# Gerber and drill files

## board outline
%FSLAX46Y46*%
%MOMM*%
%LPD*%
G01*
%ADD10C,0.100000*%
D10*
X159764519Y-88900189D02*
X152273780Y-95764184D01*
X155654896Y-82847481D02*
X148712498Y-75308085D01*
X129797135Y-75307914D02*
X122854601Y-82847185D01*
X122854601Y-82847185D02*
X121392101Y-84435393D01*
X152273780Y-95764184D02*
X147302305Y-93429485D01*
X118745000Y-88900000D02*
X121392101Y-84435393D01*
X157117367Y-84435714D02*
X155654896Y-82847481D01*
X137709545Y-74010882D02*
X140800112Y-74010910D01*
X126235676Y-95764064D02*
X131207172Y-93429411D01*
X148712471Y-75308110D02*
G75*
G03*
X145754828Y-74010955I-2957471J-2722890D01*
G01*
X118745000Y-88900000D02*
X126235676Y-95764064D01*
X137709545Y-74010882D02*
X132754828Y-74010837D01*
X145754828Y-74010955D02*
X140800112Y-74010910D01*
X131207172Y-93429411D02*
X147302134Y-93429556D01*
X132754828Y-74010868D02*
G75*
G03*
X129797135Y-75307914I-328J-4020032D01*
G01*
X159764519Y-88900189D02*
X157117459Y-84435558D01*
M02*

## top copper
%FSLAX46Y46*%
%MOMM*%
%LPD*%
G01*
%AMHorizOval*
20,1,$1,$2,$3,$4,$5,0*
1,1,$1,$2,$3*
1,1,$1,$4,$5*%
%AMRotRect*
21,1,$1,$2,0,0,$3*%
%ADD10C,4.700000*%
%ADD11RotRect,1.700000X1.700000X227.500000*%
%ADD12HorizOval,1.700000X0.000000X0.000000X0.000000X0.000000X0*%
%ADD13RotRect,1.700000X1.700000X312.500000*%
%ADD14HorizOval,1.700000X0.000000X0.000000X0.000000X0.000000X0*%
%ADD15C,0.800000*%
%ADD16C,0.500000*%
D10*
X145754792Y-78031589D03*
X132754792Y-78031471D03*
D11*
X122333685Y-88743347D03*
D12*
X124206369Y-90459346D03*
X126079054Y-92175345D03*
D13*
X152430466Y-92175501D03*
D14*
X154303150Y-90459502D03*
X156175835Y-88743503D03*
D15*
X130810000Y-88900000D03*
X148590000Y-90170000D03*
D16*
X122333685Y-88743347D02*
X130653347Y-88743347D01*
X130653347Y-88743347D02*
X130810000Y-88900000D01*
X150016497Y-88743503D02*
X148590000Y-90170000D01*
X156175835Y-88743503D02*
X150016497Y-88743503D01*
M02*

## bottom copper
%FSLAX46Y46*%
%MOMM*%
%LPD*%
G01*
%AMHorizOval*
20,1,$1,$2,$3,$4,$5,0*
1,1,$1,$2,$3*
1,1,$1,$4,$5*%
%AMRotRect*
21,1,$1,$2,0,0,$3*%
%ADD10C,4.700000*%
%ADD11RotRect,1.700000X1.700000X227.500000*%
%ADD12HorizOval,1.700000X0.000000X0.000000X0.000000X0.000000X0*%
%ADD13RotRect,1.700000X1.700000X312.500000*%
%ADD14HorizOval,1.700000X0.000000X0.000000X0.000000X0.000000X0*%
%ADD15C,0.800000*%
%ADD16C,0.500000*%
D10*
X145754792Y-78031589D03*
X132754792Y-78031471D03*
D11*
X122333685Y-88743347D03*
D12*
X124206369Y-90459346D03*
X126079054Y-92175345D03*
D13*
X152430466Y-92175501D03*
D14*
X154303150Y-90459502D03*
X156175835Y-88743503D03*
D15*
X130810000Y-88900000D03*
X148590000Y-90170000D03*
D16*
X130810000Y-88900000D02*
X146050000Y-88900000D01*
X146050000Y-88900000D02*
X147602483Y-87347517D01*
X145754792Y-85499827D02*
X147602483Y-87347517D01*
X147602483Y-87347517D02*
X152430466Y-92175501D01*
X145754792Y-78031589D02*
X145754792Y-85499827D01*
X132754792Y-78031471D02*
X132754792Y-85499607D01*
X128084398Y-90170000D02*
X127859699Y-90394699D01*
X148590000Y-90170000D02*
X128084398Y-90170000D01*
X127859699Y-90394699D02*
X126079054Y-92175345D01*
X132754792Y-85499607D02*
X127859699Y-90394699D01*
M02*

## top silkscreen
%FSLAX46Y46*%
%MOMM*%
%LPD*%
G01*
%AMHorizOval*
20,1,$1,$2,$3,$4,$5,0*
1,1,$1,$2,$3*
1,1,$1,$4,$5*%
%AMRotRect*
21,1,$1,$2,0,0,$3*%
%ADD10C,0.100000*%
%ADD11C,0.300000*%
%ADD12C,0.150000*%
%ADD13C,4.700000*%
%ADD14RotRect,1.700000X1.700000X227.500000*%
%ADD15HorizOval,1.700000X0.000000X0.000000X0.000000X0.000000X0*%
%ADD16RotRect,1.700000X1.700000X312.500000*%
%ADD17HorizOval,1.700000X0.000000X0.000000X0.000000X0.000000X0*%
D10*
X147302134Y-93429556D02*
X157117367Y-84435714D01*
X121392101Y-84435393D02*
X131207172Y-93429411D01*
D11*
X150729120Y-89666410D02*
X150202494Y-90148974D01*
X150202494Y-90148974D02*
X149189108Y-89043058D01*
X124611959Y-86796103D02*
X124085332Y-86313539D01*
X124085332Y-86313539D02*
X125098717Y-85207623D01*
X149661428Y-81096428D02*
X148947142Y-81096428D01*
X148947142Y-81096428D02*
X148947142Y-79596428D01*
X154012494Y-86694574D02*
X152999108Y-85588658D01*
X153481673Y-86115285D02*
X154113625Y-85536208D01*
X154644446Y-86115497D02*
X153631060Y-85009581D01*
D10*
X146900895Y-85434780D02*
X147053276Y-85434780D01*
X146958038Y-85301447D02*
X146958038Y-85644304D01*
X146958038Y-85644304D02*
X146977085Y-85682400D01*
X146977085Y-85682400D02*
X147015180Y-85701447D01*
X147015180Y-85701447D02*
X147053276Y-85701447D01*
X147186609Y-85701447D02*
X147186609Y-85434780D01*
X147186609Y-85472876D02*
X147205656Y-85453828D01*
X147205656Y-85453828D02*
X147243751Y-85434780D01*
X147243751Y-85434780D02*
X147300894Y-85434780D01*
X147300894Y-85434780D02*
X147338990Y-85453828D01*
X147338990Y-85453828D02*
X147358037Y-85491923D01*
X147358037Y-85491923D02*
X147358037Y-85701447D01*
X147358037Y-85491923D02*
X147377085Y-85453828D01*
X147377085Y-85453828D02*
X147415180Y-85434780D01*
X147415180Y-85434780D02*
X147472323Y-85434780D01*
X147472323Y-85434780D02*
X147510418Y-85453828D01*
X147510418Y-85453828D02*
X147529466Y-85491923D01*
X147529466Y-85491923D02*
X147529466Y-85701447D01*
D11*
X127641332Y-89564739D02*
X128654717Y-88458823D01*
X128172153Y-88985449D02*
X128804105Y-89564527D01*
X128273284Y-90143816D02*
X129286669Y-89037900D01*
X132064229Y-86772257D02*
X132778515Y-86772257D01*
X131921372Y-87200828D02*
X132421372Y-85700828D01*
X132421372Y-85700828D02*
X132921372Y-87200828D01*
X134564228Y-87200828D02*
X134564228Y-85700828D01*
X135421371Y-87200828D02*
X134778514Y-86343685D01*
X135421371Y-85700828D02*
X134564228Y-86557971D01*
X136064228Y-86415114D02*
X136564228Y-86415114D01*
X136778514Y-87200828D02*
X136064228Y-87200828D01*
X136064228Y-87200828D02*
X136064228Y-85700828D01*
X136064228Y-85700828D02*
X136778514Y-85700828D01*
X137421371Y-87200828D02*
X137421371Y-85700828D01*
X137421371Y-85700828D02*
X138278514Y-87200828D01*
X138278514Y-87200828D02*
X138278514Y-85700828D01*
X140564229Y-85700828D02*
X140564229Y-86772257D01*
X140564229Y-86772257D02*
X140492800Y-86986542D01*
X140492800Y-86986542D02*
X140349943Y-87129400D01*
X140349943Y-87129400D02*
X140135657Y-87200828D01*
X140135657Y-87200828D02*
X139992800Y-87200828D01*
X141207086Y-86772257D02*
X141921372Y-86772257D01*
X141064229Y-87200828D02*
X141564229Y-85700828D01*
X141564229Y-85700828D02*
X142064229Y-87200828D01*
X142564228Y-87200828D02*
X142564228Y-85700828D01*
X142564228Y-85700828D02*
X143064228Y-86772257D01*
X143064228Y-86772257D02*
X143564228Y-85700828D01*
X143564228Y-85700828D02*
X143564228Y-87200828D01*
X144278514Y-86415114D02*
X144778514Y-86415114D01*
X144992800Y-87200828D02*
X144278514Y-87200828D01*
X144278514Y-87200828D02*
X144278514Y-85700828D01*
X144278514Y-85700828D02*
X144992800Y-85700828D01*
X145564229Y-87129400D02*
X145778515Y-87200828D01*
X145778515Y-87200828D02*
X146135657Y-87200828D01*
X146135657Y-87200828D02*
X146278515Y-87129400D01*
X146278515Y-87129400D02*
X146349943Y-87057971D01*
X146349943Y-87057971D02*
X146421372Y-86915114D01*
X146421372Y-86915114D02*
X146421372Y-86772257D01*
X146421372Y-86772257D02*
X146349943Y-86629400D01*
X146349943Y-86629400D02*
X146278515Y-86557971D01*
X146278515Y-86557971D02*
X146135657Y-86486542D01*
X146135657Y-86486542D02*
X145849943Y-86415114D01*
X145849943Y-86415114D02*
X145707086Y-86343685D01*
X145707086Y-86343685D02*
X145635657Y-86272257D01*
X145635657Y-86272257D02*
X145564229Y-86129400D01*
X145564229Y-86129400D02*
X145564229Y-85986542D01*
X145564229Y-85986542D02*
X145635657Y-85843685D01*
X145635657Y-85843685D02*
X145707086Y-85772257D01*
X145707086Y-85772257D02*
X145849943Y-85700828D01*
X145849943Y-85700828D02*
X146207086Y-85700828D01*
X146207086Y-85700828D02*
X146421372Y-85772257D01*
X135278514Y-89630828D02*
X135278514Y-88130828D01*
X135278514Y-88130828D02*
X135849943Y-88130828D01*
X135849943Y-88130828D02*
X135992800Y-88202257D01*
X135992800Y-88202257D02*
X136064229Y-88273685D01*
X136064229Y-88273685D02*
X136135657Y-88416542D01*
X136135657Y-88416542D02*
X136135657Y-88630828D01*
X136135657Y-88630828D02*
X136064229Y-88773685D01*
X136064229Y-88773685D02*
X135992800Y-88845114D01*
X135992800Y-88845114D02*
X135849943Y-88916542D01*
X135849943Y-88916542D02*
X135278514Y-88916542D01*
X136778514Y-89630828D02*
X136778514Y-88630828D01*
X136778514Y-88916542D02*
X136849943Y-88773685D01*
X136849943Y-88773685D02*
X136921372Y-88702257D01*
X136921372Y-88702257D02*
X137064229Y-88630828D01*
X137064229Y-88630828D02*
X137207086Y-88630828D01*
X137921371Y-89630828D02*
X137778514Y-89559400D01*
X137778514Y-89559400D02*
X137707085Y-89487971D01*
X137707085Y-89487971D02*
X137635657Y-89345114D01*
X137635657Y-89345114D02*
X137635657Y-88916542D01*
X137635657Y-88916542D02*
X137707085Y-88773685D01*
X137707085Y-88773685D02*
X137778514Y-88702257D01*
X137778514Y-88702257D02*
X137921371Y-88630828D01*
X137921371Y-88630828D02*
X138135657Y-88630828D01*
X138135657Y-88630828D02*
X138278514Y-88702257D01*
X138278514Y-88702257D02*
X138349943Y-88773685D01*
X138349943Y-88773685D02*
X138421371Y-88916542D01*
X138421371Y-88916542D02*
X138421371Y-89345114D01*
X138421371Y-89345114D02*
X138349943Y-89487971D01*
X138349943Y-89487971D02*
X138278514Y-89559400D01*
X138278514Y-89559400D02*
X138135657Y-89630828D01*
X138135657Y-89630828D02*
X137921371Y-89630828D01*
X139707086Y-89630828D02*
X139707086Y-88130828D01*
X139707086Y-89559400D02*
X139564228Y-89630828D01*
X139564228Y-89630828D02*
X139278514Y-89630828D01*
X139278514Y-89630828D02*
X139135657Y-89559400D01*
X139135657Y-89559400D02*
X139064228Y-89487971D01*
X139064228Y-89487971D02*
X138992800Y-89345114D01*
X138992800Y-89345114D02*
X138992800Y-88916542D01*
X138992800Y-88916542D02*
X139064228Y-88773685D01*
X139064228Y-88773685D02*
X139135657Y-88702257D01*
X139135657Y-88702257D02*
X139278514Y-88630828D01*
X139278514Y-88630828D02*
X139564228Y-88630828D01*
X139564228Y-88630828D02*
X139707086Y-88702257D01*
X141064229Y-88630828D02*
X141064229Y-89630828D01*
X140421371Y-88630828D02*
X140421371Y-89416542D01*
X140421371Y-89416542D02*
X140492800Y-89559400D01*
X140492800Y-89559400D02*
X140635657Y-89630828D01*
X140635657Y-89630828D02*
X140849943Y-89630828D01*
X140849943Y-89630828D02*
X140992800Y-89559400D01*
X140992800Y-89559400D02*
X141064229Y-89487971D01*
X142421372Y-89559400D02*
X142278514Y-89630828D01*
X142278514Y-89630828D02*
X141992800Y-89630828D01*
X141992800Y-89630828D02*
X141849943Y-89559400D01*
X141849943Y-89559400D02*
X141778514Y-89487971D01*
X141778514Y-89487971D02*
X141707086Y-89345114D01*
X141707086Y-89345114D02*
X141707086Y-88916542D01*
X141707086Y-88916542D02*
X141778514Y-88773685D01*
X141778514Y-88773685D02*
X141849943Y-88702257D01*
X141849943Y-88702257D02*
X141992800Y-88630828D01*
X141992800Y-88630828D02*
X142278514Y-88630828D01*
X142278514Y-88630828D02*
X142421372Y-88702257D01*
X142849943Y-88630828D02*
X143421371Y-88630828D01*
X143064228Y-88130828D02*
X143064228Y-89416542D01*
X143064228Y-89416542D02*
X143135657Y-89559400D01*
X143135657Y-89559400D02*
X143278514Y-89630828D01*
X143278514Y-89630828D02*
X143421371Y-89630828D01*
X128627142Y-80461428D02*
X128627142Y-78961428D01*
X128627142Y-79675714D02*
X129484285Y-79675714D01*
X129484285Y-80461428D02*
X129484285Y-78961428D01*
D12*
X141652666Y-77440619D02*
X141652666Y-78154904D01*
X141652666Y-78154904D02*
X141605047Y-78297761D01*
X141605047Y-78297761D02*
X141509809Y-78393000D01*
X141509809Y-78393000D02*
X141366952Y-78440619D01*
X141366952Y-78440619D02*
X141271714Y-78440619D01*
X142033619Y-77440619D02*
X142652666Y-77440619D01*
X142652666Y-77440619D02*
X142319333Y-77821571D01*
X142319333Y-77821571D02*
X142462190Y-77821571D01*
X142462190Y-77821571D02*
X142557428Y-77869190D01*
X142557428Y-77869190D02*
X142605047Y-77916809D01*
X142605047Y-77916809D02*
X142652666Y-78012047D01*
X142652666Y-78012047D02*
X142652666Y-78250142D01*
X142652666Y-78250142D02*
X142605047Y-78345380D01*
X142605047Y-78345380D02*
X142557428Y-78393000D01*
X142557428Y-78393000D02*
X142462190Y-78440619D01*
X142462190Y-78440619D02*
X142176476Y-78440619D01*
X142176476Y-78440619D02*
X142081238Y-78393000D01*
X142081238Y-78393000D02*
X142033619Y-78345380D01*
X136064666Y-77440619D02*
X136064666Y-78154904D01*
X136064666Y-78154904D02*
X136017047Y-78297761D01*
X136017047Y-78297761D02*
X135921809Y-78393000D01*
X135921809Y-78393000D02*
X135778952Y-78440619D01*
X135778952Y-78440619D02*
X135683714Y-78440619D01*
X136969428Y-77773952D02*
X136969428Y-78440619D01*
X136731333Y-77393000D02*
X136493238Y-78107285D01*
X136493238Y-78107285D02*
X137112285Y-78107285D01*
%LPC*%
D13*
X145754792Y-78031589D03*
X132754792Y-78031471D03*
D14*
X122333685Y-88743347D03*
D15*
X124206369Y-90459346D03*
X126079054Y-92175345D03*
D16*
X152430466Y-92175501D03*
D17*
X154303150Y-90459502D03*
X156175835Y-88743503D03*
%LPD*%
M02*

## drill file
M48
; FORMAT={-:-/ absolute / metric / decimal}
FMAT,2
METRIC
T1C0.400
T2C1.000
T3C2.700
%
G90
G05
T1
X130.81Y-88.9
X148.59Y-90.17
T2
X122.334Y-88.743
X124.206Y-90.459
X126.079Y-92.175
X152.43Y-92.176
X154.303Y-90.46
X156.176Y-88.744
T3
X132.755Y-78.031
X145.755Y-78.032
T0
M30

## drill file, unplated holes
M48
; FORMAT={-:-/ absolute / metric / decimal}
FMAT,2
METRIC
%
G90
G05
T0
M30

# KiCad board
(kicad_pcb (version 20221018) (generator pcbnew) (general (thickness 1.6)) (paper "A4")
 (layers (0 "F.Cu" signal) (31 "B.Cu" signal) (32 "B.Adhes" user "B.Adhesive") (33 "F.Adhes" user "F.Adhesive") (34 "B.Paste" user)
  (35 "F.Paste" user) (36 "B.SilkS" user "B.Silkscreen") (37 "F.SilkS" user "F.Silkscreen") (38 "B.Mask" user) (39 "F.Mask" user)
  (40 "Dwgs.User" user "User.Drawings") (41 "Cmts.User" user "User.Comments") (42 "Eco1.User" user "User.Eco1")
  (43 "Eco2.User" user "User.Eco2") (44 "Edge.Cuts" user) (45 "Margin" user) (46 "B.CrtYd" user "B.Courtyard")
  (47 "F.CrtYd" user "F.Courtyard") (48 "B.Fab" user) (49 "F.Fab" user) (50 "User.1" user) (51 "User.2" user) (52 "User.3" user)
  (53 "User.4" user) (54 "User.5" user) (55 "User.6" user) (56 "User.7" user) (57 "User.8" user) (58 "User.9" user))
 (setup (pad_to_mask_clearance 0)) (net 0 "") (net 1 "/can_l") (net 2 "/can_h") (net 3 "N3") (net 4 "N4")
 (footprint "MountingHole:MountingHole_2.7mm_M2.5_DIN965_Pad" (layer "F.Cu") (at 145.754792 78.031589)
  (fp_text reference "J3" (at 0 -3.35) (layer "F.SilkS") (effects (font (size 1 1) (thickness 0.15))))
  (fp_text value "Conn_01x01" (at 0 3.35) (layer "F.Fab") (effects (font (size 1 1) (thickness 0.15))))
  (pad "1" thru_hole circle (at 0 0) (size 4.7 4.7) (drill 2.7) (layers "*.Cu" "*.Mask") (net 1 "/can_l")))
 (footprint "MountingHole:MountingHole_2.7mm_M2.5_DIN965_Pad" (layer "F.Cu") (at 132.754792 78.031471)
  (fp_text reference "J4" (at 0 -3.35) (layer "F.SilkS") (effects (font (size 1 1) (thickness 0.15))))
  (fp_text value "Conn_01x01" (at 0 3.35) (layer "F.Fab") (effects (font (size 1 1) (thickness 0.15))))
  (pad "1" thru_hole circle (at 0 0) (size 4.7 4.7) (drill 2.7) (layers "*.Cu" "*.Mask") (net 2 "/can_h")))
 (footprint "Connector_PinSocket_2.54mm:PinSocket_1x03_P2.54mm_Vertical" (layer "B.Cu") (at 122.333685 88.743347 -132.5)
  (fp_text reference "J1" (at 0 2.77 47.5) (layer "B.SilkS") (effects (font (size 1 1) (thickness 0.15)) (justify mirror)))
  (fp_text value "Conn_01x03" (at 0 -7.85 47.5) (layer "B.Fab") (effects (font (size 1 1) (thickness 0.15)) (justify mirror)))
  (pad "1" thru_hole rect (at 0 0 227.5) (size 1.7 1.7) (drill 1) (layers "*.Cu" "*.Mask") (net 1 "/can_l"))
  (pad "2" thru_hole oval (at 0 -2.54 227.5) (size 1.7 1.7) (drill 1) (layers "*.Cu" "*.Mask") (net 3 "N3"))
  (pad "3" thru_hole oval (at 0 -5.08 227.5) (size 1.7 1.7) (drill 1) (layers "*.Cu" "*.Mask") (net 2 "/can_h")))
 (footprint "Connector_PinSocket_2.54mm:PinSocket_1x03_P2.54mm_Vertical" (layer "B.Cu") (at 152.430466 92.175501 -47.5)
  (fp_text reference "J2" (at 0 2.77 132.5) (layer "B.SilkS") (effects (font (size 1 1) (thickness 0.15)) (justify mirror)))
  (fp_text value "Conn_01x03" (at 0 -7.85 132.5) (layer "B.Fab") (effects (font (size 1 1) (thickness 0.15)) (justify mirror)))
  (pad "1" thru_hole rect (at 0 0 312.5) (size 1.7 1.7) (drill 1) (layers "*.Cu" "*.Mask") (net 1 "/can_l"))
  (pad "2" thru_hole oval (at 0 -2.54 312.5) (size 1.7 1.7) (drill 1) (layers "*.Cu" "*.Mask") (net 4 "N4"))
  (pad "3" thru_hole oval (at 0 -5.08 312.5) (size 1.7 1.7) (drill 1) (layers "*.Cu" "*.Mask") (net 2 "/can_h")))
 (gr_line (start 147.302134 93.429556) (end 157.117367 84.435714) (stroke (width 0.1) (type solid)) (layer "F.SilkS"))
 (gr_line (start 121.392101 84.435393) (end 131.207172 93.429411) (stroke (width 0.1) (type solid)) (layer "F.SilkS"))
 (gr_line (start 159.764519 88.900189) (end 152.27378 95.764184) (stroke (width 0.1) (type solid)) (layer "Edge.Cuts"))
 (gr_line (start 155.654896 82.847481) (end 148.712498 75.308085) (stroke (width 0.1) (type solid)) (layer "Edge.Cuts"))
 (gr_line (start 129.797135 75.307914) (end 122.854601 82.847185) (stroke (width 0.1) (type solid)) (layer "Edge.Cuts"))
 (gr_line (start 122.854601 82.847185) (end 121.392101 84.435393) (stroke (width 0.1) (type solid)) (layer "Edge.Cuts"))
 (gr_line (start 152.27378 95.764184) (end 147.302305 93.429485) (stroke (width 0.1) (type solid)) (layer "Edge.Cuts"))
 (gr_line (start 118.745 88.9) (end 121.392101 84.435393) (stroke (width 0.1) (type solid)) (layer "Edge.Cuts"))
 (gr_line (start 157.117367 84.435714) (end 155.654896 82.847481) (stroke (width 0.1) (type solid)) (layer "Edge.Cuts"))
 (gr_line (start 137.709545 74.010882) (end 140.800112 74.01091) (stroke (width 0.1) (type solid)) (layer "Edge.Cuts"))
 (gr_line (start 126.235676 95.764064) (end 131.207172 93.429411) (stroke (width 0.1) (type solid)) (layer "Edge.Cuts"))
 (gr_arc (start 145.754828 74.010955) (mid 147.369649 74.349449) (end 148.712498 75.308085) (stroke (width 0.1) (type solid))
  (layer "Edge.Cuts"))
 (gr_line (start 118.745 88.9) (end 126.235676 95.764064) (stroke (width 0.1) (type solid)) (layer "Edge.Cuts"))
 (gr_line (start 137.709545 74.010882) (end 132.754828 74.010837) (stroke (width 0.1) (type solid)) (layer "Edge.Cuts"))
 (gr_line (start 145.754828 74.010955) (end 140.800112 74.01091) (stroke (width 0.1) (type solid)) (layer "Edge.Cuts"))
 (gr_line (start 131.207172 93.429411) (end 147.302134 93.429556) (stroke (width 0.1) (type solid)) (layer "Edge.Cuts"))
 (gr_arc (start 129.797135 75.307914) (mid 131.140001 74.349302) (end 132.754828 74.010837) (stroke (width 0.1) (type solid))
  (layer "Edge.Cuts"))
 (gr_line (start 159.764519 88.900189) (end 157.117459 84.435558) (stroke (width 0.1) (type solid)) (layer "Edge.Cuts"))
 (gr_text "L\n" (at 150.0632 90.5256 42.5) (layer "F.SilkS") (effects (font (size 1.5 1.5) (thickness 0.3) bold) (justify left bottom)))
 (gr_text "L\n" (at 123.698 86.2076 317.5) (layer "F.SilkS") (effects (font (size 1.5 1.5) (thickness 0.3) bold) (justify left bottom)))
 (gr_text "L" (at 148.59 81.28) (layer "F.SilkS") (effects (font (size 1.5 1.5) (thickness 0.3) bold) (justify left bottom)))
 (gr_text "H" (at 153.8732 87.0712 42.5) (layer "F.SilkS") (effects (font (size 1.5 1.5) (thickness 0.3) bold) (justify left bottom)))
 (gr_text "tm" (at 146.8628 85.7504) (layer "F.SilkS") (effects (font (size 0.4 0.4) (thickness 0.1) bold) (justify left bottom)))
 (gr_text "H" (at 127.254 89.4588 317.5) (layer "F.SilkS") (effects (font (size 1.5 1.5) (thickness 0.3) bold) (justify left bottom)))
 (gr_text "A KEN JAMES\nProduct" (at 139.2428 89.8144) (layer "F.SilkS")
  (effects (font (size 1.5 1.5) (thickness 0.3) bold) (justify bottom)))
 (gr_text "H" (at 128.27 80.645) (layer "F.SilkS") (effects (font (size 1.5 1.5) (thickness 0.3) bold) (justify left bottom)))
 (segment (start 122.333685 88.743347) (end 130.653347 88.743347) (width 0.5) (layer "F.Cu") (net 1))
 (segment (start 130.653347 88.743347) (end 130.81 88.9) (width 0.5) (layer "F.Cu") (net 1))
 (via (at 130.81 88.9) (size 0.8) (drill 0.4) (layers "F.Cu" "B.Cu") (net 1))
 (segment (start 130.81 88.9) (end 146.05 88.9) (width 0.5) (layer "B.Cu") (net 1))
 (segment (start 146.05 88.9) (end 147.602483 87.347517) (width 0.5) (layer "B.Cu") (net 1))
 (segment (start 145.754792 85.499827) (end 147.602483 87.347517) (width 0.5) (layer "B.Cu") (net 1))
 (segment (start 147.602483 87.347517) (end 152.430466 92.175501) (width 0.5) (layer "B.Cu") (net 1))
 (segment (start 145.754792 78.031589) (end 145.754792 85.499827) (width 0.5) (layer "B.Cu") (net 1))
 (segment (start 150.016497 88.743503) (end 148.59 90.17) (width 0.5) (layer "F.Cu") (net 2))
 (segment (start 156.175835 88.743503) (end 150.016497 88.743503) (width 0.5) (layer "F.Cu") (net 2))
 (via (at 148.59 90.17) (size 0.8) (drill 0.4) (layers "F.Cu" "B.Cu") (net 2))
 (segment (start 132.754792 78.031471) (end 132.754792 85.499607) (width 0.5) (layer "B.Cu") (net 2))
 (segment (start 128.084398 90.17) (end 127.859699 90.394699) (width 0.5) (layer "B.Cu") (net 2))
 (segment (start 148.59 90.17) (end 128.084398 90.17) (width 0.5) (layer "B.Cu") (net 2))
 (segment (start 127.859699 90.394699) (end 126.079054 92.175345) (width 0.5) (layer "B.Cu") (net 2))
 (segment (start 132.754792 85.499607) (end 127.859699 90.394699) (width 0.5) (layer "B.Cu") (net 2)))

